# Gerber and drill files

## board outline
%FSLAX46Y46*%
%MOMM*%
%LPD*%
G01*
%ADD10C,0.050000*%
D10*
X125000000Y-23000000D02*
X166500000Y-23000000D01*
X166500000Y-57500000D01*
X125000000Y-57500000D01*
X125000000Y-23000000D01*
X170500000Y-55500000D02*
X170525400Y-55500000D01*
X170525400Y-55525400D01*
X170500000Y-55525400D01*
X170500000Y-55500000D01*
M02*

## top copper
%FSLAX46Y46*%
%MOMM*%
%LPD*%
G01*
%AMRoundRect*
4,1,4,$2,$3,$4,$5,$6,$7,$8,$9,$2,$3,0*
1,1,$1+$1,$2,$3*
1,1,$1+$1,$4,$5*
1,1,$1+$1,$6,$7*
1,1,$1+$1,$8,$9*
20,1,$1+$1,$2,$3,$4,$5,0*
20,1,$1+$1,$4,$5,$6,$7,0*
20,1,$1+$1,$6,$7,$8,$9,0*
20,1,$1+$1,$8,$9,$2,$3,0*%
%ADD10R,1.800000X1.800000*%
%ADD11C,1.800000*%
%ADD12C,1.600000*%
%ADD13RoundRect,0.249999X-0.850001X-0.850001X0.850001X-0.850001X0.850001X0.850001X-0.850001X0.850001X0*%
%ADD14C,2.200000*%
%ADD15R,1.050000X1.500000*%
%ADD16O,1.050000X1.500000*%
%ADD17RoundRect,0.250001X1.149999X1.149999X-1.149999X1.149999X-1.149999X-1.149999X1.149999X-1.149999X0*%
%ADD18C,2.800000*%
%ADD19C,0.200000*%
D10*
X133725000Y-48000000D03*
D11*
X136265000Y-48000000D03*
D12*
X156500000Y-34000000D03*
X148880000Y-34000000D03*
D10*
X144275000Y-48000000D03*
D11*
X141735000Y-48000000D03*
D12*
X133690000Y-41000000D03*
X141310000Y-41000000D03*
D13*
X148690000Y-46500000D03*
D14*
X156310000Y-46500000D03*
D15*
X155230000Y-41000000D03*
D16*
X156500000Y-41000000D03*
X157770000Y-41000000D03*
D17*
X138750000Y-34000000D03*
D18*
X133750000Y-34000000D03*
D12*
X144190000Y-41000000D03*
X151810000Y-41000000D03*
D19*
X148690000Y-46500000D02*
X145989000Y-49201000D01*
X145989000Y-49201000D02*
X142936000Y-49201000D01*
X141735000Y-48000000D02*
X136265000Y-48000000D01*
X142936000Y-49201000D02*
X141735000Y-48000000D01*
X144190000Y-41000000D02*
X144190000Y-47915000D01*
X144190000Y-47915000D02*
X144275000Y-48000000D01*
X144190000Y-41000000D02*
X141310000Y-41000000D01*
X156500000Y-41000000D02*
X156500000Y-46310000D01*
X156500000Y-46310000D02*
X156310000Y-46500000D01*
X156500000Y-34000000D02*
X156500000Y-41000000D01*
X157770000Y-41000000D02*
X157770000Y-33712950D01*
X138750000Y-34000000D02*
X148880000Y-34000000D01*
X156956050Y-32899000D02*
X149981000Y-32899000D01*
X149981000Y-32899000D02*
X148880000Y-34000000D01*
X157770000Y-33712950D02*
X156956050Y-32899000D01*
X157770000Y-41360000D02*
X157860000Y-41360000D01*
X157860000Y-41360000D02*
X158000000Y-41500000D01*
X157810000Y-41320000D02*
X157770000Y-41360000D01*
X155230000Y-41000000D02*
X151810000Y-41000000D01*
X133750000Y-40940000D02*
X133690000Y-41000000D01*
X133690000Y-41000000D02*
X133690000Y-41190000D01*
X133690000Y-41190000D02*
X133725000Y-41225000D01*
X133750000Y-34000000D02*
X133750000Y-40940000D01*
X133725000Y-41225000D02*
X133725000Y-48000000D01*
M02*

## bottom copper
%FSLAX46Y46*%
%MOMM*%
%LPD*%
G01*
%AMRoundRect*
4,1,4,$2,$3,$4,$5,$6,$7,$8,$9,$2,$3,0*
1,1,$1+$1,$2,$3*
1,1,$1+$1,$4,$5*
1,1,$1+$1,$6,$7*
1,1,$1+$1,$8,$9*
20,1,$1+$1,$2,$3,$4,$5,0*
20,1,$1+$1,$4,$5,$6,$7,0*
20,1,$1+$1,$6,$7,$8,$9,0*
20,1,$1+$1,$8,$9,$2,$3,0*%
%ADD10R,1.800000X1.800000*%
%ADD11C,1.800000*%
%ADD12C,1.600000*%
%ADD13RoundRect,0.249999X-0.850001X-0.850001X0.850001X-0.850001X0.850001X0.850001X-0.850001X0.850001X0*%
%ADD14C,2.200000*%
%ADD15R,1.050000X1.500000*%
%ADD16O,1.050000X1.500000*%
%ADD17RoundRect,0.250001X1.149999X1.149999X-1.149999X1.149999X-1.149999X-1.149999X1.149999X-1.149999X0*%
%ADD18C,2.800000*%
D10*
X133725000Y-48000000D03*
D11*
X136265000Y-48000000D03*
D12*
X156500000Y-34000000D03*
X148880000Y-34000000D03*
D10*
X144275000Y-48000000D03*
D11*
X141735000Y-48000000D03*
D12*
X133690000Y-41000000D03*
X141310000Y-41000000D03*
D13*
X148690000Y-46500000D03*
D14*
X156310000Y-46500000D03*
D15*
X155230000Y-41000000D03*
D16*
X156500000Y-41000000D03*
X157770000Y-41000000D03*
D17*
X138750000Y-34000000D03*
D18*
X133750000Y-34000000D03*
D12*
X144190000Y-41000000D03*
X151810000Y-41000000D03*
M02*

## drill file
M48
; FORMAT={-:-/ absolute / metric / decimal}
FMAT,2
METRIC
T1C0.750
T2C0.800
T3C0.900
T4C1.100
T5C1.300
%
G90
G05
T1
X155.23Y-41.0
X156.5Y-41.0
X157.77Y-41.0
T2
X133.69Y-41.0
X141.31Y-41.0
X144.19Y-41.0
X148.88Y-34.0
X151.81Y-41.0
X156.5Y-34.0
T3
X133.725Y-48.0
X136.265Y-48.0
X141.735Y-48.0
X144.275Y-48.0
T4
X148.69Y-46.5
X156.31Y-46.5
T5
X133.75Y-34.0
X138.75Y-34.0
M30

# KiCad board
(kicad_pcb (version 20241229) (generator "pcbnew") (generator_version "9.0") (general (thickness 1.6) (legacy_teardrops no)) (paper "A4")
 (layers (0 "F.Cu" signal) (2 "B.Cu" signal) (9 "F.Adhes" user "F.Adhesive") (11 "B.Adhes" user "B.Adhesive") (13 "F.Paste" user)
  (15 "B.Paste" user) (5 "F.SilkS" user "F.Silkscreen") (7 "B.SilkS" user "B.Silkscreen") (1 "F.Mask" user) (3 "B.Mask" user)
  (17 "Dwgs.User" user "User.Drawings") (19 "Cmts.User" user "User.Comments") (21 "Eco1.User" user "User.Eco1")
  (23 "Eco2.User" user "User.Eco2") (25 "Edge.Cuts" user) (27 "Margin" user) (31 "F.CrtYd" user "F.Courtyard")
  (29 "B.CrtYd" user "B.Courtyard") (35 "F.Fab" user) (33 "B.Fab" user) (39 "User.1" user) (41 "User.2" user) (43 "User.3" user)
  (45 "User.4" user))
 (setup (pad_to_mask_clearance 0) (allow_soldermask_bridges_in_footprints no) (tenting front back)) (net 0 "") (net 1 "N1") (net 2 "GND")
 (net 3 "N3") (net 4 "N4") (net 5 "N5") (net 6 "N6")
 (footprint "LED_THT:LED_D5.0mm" (layer "F.Cu") (at 133.725 48)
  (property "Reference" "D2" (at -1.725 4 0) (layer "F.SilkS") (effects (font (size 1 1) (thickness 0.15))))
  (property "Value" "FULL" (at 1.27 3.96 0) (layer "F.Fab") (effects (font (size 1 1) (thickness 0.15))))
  (pad "1" thru_hole rect (at 0 0) (size 1.8 1.8) (drill 0.9) (layers "*.Cu" "*.Mask") (remove_unused_layers no) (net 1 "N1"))
  (pad "2" thru_hole circle (at 2.54 0) (size 1.8 1.8) (drill 0.9) (layers "*.Cu" "*.Mask") (remove_unused_layers no) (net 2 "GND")))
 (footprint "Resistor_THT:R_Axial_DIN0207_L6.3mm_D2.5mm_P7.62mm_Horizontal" (layer "F.Cu") (at 156.5 34 180)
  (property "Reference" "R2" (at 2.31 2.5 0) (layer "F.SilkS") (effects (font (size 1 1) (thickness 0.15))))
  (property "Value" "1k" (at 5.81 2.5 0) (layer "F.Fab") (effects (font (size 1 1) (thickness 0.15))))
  (pad "1" thru_hole circle (at 0 0 180) (size 1.6 1.6) (drill 0.8) (layers "*.Cu" "*.Mask") (remove_unused_layers no) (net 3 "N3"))
  (pad "2" thru_hole circle (at 7.62 0 180) (size 1.6 1.6) (drill 0.8) (layers "*.Cu" "*.Mask") (remove_unused_layers no) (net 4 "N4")))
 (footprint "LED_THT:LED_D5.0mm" (layer "F.Cu") (at 144.275 48 180)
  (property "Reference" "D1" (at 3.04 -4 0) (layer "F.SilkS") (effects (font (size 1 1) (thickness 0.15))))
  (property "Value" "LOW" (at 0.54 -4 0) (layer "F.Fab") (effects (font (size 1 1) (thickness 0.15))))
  (pad "1" thru_hole rect (at 0 0 180) (size 1.8 1.8) (drill 0.9) (layers "*.Cu" "*.Mask") (remove_unused_layers no) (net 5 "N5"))
  (pad "2" thru_hole circle (at 2.54 0 180) (size 1.8 1.8) (drill 0.9) (layers "*.Cu" "*.Mask") (remove_unused_layers no) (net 2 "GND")))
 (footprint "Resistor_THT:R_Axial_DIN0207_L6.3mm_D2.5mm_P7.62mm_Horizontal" (layer "F.Cu") (at 133.69 41)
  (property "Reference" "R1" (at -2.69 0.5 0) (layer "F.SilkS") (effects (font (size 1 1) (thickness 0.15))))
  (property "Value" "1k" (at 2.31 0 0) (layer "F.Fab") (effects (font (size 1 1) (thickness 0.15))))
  (pad "1" thru_hole circle (at 0 0) (size 1.6 1.6) (drill 0.8) (layers "*.Cu" "*.Mask") (remove_unused_layers no) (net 1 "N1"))
  (pad "2" thru_hole circle (at 7.62 0) (size 1.6 1.6) (drill 0.8) (layers "*.Cu" "*.Mask") (remove_unused_layers no) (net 5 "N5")))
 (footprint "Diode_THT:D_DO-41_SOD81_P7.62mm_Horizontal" (layer "F.Cu") (at 148.69 46.5)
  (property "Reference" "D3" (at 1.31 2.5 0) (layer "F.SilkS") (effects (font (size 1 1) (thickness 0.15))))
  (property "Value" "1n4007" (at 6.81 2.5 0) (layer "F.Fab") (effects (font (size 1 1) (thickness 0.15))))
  (pad "1" thru_hole roundrect (at 0 0) (size 2.2 2.2) (drill 1.1) (layers "*.Cu" "*.Mask") (remove_unused_layers no)
   (roundrect_rratio 0.113636) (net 2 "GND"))
  (pad "2" thru_hole circle (at 7.62 0) (size 2.2 2.2) (drill 1.1) (layers "*.Cu" "*.Mask") (remove_unused_layers no) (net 3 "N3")))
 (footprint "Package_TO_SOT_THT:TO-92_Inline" (layer "F.Cu") (at 155.23 41)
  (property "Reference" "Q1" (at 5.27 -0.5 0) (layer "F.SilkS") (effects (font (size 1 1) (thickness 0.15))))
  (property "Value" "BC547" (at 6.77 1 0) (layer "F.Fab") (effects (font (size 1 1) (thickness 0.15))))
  (pad "1" thru_hole rect (at 0 0) (size 1.05 1.5) (drill 0.75) (layers "*.Cu" "*.Mask") (remove_unused_layers no) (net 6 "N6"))
  (pad "2" thru_hole oval (at 1.27 0) (size 1.05 1.5) (drill 0.75) (layers "*.Cu" "*.Mask") (remove_unused_layers no) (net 3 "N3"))
  (pad "3" thru_hole oval (at 2.54 0) (size 1.05 1.5) (drill 0.75) (layers "*.Cu" "*.Mask") (remove_unused_layers no) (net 4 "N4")))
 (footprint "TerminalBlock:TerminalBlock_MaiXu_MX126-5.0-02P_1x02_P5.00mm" (layer "F.Cu") (at 138.75 34 180)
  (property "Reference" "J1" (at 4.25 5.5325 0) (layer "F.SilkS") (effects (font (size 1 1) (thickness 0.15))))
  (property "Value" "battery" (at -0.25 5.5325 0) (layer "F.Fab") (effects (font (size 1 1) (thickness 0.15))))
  (pad "1" thru_hole roundrect (at 0 0 180) (size 2.8 2.8) (drill 1.3) (layers "*.Cu" "*.Mask") (remove_unused_layers no)
   (roundrect_rratio 0.089286) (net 4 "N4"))
  (pad "2" thru_hole circle (at 5 0 180) (size 2.8 2.8) (drill 1.3) (layers "*.Cu" "*.Mask") (remove_unused_layers no) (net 1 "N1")))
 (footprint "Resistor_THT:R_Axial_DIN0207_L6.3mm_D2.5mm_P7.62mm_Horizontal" (layer "F.Cu") (at 144.19 41)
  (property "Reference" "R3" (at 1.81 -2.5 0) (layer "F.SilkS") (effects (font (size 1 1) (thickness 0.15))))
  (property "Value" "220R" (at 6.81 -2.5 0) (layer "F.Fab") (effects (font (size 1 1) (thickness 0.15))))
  (pad "1" thru_hole circle (at 0 0) (size 1.6 1.6) (drill 0.8) (layers "*.Cu" "*.Mask") (remove_unused_layers no) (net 5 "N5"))
  (pad "2" thru_hole circle (at 7.62 0) (size 1.6 1.6) (drill 0.8) (layers "*.Cu" "*.Mask") (remove_unused_layers no) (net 6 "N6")))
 (gr_rect (start 125 23) (end 166.5 57.5) (stroke (width 0.05) (type default)) (fill no) (layer "Edge.Cuts"))
 (gr_rect (start 170.5 55.5) (end 170.5254 55.5254) (stroke (width 0.05) (type default)) (fill no) (layer "Edge.Cuts"))
 (segment (start 148.69 46.5) (end 145.989 49.201) (width 0.2) (layer "F.Cu") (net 2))
 (segment (start 145.989 49.201) (end 142.936 49.201) (width 0.2) (layer "F.Cu") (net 2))
 (segment (start 141.735 48) (end 136.265 48) (width 0.2) (layer "F.Cu") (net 2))
 (segment (start 142.936 49.201) (end 141.735 48) (width 0.2) (layer "F.Cu") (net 2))
 (segment (start 144.19 41) (end 144.19 47.915) (width 0.2) (layer "F.Cu") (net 5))
 (segment (start 144.19 47.915) (end 144.275 48) (width 0.2) (layer "F.Cu") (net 5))
 (segment (start 144.19 41) (end 141.31 41) (width 0.2) (layer "F.Cu") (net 5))
 (segment (start 156.5 41) (end 156.5 46.31) (width 0.2) (layer "F.Cu") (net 3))
 (segment (start 156.5 46.31) (end 156.31 46.5) (width 0.2) (layer "F.Cu") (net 3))
 (segment (start 156.5 34) (end 156.5 41) (width 0.2) (layer "F.Cu") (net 3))
 (segment (start 157.77 41) (end 157.77 33.71295) (width 0.2) (layer "F.Cu") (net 4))
 (segment (start 138.75 34) (end 148.88 34) (width 0.2) (layer "F.Cu") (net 4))
 (segment (start 156.95605 32.899) (end 149.981 32.899) (width 0.2) (layer "F.Cu") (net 4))
 (segment (start 149.981 32.899) (end 148.88 34) (width 0.2) (layer "F.Cu") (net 4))
 (segment (start 157.77 33.71295) (end 156.95605 32.899) (width 0.2) (layer "F.Cu") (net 4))
 (segment (start 157.77 41.36) (end 157.86 41.36) (width 0.2) (layer "F.Cu") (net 4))
 (segment (start 157.86 41.36) (end 158 41.5) (width 0.2) (layer "F.Cu") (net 4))
 (segment (start 157.81 41.32) (end 157.77 41.36) (width 0.2) (layer "F.Cu") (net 4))
 (segment (start 155.23 41) (end 151.81 41) (width 0.2) (layer "F.Cu") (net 6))
 (segment (start 133.75 40.94) (end 133.69 41) (width 0.2) (layer "F.Cu") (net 1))
 (segment (start 133.69 41) (end 133.69 41.19) (width 0.2) (layer "F.Cu") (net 1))
 (segment (start 133.69 41.19) (end 133.725 41.225) (width 0.2) (layer "F.Cu") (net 1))
 (segment (start 133.75 34) (end 133.75 40.94) (width 0.2) (layer "F.Cu") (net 1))
 (segment (start 133.725 41.225) (end 133.725 48) (width 0.2) (layer "F.Cu") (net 1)))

